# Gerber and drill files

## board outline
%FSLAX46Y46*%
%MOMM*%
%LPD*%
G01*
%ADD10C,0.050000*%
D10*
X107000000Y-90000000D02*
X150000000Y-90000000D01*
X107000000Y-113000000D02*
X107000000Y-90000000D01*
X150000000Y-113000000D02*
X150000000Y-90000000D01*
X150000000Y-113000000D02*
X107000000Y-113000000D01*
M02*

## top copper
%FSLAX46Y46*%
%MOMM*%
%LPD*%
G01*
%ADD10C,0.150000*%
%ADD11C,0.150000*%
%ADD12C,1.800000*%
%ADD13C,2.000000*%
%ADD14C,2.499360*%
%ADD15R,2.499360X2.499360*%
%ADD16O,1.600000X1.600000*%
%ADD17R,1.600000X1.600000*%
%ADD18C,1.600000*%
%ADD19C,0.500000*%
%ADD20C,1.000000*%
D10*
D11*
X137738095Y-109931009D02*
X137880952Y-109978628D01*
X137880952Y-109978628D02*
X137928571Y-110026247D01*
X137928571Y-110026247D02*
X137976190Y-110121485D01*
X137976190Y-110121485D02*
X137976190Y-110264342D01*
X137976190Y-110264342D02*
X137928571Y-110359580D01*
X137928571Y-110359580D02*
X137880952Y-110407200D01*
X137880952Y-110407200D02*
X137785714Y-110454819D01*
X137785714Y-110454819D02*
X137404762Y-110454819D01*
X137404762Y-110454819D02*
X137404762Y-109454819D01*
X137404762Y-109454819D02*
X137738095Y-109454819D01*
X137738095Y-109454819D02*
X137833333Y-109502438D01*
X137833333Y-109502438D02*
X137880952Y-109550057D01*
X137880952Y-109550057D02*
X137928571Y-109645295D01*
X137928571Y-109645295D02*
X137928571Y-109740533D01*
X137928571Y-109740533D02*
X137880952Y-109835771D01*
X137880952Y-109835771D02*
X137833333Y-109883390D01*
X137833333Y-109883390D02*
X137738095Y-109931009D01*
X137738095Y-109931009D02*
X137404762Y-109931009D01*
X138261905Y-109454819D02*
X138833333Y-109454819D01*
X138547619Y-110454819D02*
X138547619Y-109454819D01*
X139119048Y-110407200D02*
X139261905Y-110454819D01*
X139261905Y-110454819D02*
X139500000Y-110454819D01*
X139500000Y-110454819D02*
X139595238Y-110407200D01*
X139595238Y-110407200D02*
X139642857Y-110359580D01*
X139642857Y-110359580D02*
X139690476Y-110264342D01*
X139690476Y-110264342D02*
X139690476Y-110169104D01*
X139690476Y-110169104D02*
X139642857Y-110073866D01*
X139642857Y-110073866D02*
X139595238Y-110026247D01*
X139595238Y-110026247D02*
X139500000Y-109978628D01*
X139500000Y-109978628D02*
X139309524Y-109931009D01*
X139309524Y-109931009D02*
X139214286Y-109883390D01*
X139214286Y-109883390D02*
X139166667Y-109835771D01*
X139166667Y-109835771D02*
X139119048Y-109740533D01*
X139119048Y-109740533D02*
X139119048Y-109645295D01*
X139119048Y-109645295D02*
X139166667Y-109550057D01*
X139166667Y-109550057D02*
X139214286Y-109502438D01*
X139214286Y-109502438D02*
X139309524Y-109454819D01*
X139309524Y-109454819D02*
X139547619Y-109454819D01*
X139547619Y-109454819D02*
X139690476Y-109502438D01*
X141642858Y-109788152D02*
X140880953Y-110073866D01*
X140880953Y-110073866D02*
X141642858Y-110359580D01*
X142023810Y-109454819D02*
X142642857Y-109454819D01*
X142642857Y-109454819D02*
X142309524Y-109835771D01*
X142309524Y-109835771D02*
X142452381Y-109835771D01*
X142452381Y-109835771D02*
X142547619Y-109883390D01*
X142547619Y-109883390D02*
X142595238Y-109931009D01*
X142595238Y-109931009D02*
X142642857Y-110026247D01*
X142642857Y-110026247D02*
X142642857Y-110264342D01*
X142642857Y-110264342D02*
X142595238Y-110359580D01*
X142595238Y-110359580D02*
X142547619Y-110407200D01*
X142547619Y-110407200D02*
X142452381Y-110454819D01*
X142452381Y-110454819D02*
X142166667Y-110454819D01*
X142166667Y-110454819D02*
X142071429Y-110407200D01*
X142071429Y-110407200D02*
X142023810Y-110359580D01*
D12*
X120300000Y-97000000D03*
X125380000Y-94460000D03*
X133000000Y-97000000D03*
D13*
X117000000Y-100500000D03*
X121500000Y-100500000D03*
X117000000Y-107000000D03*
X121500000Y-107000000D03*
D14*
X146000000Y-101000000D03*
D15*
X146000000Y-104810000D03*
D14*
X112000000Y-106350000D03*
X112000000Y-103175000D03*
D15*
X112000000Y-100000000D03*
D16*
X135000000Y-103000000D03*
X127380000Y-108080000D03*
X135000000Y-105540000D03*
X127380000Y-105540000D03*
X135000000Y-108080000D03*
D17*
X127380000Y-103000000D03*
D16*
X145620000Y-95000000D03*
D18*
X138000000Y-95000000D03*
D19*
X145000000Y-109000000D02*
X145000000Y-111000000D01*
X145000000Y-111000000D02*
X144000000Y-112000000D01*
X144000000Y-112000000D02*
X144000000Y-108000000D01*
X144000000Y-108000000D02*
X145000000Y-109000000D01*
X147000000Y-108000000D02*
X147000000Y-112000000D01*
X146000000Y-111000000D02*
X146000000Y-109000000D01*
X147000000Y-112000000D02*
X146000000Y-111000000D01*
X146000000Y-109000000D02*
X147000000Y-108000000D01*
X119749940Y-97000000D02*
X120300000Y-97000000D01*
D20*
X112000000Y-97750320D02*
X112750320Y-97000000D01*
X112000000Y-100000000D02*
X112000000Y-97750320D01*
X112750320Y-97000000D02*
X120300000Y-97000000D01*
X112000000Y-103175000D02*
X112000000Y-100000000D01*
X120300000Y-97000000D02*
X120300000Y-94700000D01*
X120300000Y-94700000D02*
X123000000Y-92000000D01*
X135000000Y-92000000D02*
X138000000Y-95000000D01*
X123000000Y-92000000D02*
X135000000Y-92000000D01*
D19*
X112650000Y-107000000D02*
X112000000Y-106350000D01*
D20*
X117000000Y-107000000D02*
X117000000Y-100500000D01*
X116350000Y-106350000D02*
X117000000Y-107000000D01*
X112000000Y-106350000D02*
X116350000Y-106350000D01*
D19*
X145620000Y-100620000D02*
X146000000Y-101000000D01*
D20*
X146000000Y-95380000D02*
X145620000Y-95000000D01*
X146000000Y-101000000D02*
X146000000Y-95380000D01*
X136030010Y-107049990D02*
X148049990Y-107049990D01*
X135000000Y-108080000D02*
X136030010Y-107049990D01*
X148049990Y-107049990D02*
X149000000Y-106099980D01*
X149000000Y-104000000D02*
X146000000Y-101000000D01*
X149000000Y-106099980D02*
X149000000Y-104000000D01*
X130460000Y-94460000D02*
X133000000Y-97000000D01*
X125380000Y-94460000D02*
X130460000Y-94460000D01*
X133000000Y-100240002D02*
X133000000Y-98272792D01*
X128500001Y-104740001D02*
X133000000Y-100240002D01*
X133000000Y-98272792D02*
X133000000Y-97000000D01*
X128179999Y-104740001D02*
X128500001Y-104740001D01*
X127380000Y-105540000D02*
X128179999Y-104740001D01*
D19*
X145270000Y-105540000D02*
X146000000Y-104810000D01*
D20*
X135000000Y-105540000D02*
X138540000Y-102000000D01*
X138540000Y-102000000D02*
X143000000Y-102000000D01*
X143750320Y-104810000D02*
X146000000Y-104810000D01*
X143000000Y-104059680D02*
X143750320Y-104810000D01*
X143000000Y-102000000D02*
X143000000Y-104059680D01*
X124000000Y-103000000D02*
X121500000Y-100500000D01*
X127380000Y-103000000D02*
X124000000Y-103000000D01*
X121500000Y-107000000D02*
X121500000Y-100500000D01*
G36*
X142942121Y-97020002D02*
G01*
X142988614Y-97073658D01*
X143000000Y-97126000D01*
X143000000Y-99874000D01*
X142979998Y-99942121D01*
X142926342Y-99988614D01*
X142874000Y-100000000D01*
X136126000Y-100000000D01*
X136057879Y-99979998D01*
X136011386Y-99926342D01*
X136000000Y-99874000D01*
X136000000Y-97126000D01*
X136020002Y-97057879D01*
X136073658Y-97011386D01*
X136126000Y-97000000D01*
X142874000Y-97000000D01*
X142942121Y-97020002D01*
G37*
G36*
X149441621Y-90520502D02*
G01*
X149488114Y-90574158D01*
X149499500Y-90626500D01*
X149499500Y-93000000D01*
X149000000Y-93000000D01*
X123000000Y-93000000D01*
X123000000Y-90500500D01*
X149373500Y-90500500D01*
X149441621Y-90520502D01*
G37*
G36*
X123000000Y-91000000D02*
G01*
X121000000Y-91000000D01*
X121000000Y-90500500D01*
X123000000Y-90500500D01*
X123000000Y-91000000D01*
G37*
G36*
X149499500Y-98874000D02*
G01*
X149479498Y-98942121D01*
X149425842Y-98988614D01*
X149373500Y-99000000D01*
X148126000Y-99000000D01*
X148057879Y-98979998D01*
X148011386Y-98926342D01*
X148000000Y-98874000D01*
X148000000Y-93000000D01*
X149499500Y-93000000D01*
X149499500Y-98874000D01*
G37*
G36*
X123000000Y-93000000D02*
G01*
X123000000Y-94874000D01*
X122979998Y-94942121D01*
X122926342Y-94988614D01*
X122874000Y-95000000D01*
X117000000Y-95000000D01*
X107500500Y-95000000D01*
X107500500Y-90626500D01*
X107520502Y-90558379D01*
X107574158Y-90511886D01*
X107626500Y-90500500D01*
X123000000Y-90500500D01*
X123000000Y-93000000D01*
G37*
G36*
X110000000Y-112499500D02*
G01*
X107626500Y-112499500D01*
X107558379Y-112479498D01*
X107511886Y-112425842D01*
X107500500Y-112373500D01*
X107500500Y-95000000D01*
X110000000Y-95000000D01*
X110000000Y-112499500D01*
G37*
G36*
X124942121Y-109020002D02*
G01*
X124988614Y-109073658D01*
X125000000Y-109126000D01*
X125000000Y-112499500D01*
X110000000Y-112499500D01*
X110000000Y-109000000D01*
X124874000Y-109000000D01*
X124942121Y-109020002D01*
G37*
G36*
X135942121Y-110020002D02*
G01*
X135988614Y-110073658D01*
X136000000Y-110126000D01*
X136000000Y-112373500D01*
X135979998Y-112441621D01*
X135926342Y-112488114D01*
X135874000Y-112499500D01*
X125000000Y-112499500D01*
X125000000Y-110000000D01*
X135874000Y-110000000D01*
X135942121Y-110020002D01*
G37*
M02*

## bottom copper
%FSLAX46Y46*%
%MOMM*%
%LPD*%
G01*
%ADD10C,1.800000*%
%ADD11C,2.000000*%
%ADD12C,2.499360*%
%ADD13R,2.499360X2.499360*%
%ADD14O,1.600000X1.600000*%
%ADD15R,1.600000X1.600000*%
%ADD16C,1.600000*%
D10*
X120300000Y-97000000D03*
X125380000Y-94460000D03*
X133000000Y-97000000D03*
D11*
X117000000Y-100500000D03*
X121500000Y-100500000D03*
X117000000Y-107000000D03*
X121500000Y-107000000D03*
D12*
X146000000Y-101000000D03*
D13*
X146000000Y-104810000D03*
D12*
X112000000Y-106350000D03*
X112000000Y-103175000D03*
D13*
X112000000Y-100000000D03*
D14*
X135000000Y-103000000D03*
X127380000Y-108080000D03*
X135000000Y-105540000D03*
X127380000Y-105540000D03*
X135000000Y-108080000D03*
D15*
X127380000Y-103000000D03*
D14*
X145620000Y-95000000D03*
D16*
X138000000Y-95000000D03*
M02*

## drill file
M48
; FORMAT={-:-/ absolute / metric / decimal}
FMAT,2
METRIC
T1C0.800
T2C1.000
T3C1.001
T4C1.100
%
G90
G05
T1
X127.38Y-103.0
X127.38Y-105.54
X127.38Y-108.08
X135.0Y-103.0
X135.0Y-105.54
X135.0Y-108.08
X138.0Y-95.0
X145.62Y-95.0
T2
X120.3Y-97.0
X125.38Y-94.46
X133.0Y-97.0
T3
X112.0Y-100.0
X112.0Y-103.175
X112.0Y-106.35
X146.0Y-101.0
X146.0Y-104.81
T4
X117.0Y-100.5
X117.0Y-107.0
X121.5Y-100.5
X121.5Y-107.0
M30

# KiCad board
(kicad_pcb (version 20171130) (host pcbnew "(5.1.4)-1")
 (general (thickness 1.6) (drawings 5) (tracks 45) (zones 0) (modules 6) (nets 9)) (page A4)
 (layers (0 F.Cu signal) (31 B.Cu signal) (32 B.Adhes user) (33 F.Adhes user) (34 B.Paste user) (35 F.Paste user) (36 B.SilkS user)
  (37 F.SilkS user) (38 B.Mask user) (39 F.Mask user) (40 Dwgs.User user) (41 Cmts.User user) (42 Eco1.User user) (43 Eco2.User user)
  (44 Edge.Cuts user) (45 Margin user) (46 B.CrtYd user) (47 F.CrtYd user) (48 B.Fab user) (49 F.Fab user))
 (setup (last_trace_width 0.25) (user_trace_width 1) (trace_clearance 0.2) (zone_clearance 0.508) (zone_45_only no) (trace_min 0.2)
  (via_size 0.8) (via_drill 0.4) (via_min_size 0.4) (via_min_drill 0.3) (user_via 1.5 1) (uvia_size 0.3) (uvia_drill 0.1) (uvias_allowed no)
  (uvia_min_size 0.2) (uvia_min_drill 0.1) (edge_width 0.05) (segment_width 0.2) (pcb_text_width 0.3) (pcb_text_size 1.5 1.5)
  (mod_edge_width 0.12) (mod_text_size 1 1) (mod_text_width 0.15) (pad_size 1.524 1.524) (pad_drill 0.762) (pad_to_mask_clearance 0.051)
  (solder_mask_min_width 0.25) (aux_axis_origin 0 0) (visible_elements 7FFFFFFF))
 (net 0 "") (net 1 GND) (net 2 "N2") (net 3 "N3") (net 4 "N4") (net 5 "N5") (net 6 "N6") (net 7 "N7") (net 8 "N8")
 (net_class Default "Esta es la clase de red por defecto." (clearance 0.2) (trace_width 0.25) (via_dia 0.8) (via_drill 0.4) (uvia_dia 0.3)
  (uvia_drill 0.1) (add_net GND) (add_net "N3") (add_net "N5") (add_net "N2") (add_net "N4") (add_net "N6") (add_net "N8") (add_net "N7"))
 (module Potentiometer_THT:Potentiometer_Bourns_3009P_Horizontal (layer F.Cu) (at 133 97)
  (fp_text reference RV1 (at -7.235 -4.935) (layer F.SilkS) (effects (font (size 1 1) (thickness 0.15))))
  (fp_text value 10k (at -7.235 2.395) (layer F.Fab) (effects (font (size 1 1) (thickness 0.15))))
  (pad 3 thru_hole circle (at -12.7 0) (size 1.8 1.8) (drill 1) (layers *.Cu *.Mask) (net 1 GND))
  (pad 2 thru_hole circle (at -7.62 -2.54) (size 1.8 1.8) (drill 1) (layers *.Cu *.Mask) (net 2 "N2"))
  (pad 1 thru_hole circle (at 0 0) (size 1.8 1.8) (drill 1) (layers *.Cu *.Mask) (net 2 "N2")))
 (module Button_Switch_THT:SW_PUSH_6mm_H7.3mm (layer F.Cu) (at 117 107 90)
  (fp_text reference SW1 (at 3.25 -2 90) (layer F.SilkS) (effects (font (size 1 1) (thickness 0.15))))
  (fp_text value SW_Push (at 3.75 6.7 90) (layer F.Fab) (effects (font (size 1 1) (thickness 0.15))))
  (pad 1 thru_hole circle (at 6.5 0 180) (size 2 2) (drill 1.1) (layers *.Cu *.Mask) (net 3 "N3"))
  (pad 2 thru_hole circle (at 6.5 4.5 180) (size 2 2) (drill 1.1) (layers *.Cu *.Mask) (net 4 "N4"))
  (pad 1 thru_hole circle (at 0 0 180) (size 2 2) (drill 1.1) (layers *.Cu *.Mask) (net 3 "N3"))
  (pad 2 thru_hole circle (at 0 4.5 180) (size 2 2) (drill 1.1) (layers *.Cu *.Mask) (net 4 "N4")))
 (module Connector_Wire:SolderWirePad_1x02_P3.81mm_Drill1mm (layer F.Cu) (at 146 104.81 90)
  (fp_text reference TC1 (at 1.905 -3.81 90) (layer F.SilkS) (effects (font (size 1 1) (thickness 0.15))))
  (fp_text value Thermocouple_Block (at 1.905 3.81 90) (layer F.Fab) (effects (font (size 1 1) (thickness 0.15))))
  (pad 2 thru_hole circle (at 3.81 0 90) (size 2.49936 2.49936) (drill 1.00076) (layers *.Cu *.Mask) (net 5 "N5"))
  (pad 1 thru_hole rect (at 0 0 90) (size 2.49936 2.49936) (drill 1.00076) (layers *.Cu *.Mask) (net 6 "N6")))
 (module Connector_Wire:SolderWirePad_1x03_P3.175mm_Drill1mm (layer F.Cu) (at 112 100 270)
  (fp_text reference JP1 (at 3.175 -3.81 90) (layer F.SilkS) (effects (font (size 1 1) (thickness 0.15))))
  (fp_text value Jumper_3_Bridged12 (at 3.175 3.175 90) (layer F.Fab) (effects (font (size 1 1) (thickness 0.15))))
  (pad 3 thru_hole circle (at 6.35 0 270) (size 2.49936 2.49936) (drill 1.00076) (layers *.Cu *.Mask) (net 3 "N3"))
  (pad 2 thru_hole circle (at 3.175 0 270) (size 2.49936 2.49936) (drill 1.00076) (layers *.Cu *.Mask) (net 1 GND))
  (pad 1 thru_hole rect (at 0 0 270) (size 2.49936 2.49936) (drill 1.00076) (layers *.Cu *.Mask) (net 1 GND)))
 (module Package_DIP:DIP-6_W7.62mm (layer F.Cu) (at 127.38 103)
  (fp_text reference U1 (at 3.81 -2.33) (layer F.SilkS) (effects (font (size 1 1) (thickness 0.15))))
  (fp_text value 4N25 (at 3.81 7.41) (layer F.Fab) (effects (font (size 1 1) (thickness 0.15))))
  (pad 6 thru_hole oval (at 7.62 0) (size 1.6 1.6) (drill 0.8) (layers *.Cu *.Mask) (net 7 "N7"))
  (pad 3 thru_hole oval (at 0 5.08) (size 1.6 1.6) (drill 0.8) (layers *.Cu *.Mask) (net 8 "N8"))
  (pad 5 thru_hole oval (at 7.62 2.54) (size 1.6 1.6) (drill 0.8) (layers *.Cu *.Mask) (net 6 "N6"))
  (pad 2 thru_hole oval (at 0 2.54) (size 1.6 1.6) (drill 0.8) (layers *.Cu *.Mask) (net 2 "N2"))
  (pad 4 thru_hole oval (at 7.62 5.08) (size 1.6 1.6) (drill 0.8) (layers *.Cu *.Mask) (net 5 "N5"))
  (pad 1 thru_hole rect (at 0 0) (size 1.6 1.6) (drill 0.8) (layers *.Cu *.Mask) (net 4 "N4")))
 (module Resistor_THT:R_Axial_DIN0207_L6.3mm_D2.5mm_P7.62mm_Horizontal (layer F.Cu) (at 138 95)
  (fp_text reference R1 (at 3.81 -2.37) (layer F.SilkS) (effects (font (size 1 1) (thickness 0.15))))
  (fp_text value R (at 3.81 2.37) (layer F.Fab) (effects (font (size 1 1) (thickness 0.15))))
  (pad 2 thru_hole oval (at 7.62 0) (size 1.6 1.6) (drill 0.8) (layers *.Cu *.Mask) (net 5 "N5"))
  (pad 1 thru_hole circle (at 0 0) (size 1.6 1.6) (drill 0.8) (layers *.Cu *.Mask) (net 1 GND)))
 (gr_line (start 107 90) (end 150 90) (layer Edge.Cuts) (width 0.05))
 (gr_line (start 107 113) (end 107 90) (layer Edge.Cuts) (width 0.05))
 (gr_line (start 150 113) (end 150 90) (layer Edge.Cuts) (width 0.05))
 (gr_line (start 150 113) (end 107 113) (layer Edge.Cuts) (width 0.05))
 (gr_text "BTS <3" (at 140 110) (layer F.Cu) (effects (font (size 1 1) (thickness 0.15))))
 (segment (start 145 109) (end 145 111) (width 0.5) (layer F.Cu) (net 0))
 (segment (start 145 111) (end 144 112) (width 0.5) (layer F.Cu) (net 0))
 (segment (start 144 112) (end 144 108) (width 0.5) (layer F.Cu) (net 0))
 (segment (start 144 108) (end 145 109) (width 0.5) (layer F.Cu) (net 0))
 (segment (start 147 108) (end 147 112) (width 0.5) (layer F.Cu) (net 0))
 (segment (start 146 111) (end 146 109) (width 0.5) (layer F.Cu) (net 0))
 (segment (start 147 112) (end 146 111) (width 0.5) (layer F.Cu) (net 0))
 (segment (start 146 109) (end 147 108) (width 0.5) (layer F.Cu) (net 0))
 (segment (start 119.74994 97) (end 120.3 97) (width 0.5) (layer F.Cu) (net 1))
 (segment (start 112 97.75032) (end 112.75032 97) (width 1) (layer F.Cu) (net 1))
 (segment (start 112 100) (end 112 97.75032) (width 1) (layer F.Cu) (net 1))
 (segment (start 112.75032 97) (end 120.3 97) (width 1) (layer F.Cu) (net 1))
 (segment (start 112 103.175) (end 112 100) (width 1) (layer F.Cu) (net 1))
 (segment (start 120.3 97) (end 120.3 94.7) (width 1) (layer F.Cu) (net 1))
 (segment (start 120.3 94.7) (end 123 92) (width 1) (layer F.Cu) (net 1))
 (segment (start 135 92) (end 138 95) (width 1) (layer F.Cu) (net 1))
 (segment (start 123 92) (end 135 92) (width 1) (layer F.Cu) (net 1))
 (segment (start 112.65 107) (end 112 106.35) (width 0.5) (layer F.Cu) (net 3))
 (segment (start 117 107) (end 117 100.5) (width 1) (layer F.Cu) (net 3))
 (segment (start 116.35 106.35) (end 117 107) (width 1) (layer F.Cu) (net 3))
 (segment (start 112 106.35) (end 116.35 106.35) (width 1) (layer F.Cu) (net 3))
 (segment (start 145.62 100.62) (end 146 101) (width 0.5) (layer F.Cu) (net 5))
 (segment (start 146 95.38) (end 145.62 95) (width 1) (layer F.Cu) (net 5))
 (segment (start 146 101) (end 146 95.38) (width 1) (layer F.Cu) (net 5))
 (segment (start 136.03001 107.04999) (end 148.04999 107.04999) (width 1) (layer F.Cu) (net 5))
 (segment (start 135 108.08) (end 136.03001 107.04999) (width 1) (layer F.Cu) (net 5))
 (segment (start 148.04999 107.04999) (end 149 106.09998) (width 1) (layer F.Cu) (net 5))
 (segment (start 149 104) (end 146 101) (width 1) (layer F.Cu) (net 5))
 (segment (start 149 106.09998) (end 149 104) (width 1) (layer F.Cu) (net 5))
 (segment (start 130.46 94.46) (end 133 97) (width 1) (layer F.Cu) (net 2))
 (segment (start 125.38 94.46) (end 130.46 94.46) (width 1) (layer F.Cu) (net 2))
 (segment (start 133 100.240002) (end 133 98.272792) (width 1) (layer F.Cu) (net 2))
 (segment (start 128.500001 104.740001) (end 133 100.240002) (width 1) (layer F.Cu) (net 2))
 (segment (start 133 98.272792) (end 133 97) (width 1) (layer F.Cu) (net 2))
 (segment (start 128.179999 104.740001) (end 128.500001 104.740001) (width 1) (layer F.Cu) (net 2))
 (segment (start 127.38 105.54) (end 128.179999 104.740001) (width 1) (layer F.Cu) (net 2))
 (segment (start 145.27 105.54) (end 146 104.81) (width 0.5) (layer F.Cu) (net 6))
 (segment (start 135 105.54) (end 138.54 102) (width 1) (layer F.Cu) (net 6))
 (segment (start 138.54 102) (end 143 102) (width 1) (layer F.Cu) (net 6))
 (segment (start 143.75032 104.81) (end 146 104.81) (width 1) (layer F.Cu) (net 6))
 (segment (start 143 104.05968) (end 143.75032 104.81) (width 1) (layer F.Cu) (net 6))
 (segment (start 143 102) (end 143 104.05968) (width 1) (layer F.Cu) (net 6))
 (segment (start 124 103) (end 121.5 100.5) (width 1) (layer F.Cu) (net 4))
 (segment (start 127.38 103) (end 124 103) (width 1) (layer F.Cu) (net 4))
 (segment (start 121.5 107) (end 121.5 100.5) (width 1) (layer F.Cu) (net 4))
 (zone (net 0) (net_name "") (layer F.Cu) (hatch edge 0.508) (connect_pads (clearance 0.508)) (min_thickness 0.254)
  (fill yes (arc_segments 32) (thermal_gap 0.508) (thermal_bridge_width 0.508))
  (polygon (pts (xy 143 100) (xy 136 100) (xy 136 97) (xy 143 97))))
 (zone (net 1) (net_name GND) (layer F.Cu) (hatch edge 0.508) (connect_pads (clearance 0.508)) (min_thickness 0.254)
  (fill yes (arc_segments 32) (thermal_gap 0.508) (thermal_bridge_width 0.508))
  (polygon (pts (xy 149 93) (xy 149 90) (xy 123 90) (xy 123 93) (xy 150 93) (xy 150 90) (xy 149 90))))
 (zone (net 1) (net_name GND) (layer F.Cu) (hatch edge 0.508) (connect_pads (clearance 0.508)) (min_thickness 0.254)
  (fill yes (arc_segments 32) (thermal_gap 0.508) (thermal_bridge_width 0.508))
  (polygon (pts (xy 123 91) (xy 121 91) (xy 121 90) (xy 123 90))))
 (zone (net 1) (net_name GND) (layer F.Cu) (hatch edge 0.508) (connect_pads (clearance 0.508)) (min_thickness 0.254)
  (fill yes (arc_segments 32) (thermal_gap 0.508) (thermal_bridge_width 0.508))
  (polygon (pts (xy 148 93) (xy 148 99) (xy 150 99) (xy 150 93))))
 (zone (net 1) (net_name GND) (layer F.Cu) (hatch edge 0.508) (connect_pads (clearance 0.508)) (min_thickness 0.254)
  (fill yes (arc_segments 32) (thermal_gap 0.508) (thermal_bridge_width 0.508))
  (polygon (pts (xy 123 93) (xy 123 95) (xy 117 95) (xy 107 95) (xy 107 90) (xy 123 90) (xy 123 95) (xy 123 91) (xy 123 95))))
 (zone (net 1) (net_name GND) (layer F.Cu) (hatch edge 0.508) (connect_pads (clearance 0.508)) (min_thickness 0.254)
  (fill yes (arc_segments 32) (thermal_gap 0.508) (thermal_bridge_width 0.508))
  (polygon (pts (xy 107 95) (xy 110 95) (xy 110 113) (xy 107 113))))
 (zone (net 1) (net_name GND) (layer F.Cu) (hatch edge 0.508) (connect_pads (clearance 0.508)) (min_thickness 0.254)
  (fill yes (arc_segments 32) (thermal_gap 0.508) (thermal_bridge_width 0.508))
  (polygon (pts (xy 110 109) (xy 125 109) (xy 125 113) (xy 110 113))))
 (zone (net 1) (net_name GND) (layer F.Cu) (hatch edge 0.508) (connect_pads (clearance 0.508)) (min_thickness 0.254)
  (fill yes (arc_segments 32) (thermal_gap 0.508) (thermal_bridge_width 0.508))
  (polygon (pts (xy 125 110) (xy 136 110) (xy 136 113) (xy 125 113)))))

